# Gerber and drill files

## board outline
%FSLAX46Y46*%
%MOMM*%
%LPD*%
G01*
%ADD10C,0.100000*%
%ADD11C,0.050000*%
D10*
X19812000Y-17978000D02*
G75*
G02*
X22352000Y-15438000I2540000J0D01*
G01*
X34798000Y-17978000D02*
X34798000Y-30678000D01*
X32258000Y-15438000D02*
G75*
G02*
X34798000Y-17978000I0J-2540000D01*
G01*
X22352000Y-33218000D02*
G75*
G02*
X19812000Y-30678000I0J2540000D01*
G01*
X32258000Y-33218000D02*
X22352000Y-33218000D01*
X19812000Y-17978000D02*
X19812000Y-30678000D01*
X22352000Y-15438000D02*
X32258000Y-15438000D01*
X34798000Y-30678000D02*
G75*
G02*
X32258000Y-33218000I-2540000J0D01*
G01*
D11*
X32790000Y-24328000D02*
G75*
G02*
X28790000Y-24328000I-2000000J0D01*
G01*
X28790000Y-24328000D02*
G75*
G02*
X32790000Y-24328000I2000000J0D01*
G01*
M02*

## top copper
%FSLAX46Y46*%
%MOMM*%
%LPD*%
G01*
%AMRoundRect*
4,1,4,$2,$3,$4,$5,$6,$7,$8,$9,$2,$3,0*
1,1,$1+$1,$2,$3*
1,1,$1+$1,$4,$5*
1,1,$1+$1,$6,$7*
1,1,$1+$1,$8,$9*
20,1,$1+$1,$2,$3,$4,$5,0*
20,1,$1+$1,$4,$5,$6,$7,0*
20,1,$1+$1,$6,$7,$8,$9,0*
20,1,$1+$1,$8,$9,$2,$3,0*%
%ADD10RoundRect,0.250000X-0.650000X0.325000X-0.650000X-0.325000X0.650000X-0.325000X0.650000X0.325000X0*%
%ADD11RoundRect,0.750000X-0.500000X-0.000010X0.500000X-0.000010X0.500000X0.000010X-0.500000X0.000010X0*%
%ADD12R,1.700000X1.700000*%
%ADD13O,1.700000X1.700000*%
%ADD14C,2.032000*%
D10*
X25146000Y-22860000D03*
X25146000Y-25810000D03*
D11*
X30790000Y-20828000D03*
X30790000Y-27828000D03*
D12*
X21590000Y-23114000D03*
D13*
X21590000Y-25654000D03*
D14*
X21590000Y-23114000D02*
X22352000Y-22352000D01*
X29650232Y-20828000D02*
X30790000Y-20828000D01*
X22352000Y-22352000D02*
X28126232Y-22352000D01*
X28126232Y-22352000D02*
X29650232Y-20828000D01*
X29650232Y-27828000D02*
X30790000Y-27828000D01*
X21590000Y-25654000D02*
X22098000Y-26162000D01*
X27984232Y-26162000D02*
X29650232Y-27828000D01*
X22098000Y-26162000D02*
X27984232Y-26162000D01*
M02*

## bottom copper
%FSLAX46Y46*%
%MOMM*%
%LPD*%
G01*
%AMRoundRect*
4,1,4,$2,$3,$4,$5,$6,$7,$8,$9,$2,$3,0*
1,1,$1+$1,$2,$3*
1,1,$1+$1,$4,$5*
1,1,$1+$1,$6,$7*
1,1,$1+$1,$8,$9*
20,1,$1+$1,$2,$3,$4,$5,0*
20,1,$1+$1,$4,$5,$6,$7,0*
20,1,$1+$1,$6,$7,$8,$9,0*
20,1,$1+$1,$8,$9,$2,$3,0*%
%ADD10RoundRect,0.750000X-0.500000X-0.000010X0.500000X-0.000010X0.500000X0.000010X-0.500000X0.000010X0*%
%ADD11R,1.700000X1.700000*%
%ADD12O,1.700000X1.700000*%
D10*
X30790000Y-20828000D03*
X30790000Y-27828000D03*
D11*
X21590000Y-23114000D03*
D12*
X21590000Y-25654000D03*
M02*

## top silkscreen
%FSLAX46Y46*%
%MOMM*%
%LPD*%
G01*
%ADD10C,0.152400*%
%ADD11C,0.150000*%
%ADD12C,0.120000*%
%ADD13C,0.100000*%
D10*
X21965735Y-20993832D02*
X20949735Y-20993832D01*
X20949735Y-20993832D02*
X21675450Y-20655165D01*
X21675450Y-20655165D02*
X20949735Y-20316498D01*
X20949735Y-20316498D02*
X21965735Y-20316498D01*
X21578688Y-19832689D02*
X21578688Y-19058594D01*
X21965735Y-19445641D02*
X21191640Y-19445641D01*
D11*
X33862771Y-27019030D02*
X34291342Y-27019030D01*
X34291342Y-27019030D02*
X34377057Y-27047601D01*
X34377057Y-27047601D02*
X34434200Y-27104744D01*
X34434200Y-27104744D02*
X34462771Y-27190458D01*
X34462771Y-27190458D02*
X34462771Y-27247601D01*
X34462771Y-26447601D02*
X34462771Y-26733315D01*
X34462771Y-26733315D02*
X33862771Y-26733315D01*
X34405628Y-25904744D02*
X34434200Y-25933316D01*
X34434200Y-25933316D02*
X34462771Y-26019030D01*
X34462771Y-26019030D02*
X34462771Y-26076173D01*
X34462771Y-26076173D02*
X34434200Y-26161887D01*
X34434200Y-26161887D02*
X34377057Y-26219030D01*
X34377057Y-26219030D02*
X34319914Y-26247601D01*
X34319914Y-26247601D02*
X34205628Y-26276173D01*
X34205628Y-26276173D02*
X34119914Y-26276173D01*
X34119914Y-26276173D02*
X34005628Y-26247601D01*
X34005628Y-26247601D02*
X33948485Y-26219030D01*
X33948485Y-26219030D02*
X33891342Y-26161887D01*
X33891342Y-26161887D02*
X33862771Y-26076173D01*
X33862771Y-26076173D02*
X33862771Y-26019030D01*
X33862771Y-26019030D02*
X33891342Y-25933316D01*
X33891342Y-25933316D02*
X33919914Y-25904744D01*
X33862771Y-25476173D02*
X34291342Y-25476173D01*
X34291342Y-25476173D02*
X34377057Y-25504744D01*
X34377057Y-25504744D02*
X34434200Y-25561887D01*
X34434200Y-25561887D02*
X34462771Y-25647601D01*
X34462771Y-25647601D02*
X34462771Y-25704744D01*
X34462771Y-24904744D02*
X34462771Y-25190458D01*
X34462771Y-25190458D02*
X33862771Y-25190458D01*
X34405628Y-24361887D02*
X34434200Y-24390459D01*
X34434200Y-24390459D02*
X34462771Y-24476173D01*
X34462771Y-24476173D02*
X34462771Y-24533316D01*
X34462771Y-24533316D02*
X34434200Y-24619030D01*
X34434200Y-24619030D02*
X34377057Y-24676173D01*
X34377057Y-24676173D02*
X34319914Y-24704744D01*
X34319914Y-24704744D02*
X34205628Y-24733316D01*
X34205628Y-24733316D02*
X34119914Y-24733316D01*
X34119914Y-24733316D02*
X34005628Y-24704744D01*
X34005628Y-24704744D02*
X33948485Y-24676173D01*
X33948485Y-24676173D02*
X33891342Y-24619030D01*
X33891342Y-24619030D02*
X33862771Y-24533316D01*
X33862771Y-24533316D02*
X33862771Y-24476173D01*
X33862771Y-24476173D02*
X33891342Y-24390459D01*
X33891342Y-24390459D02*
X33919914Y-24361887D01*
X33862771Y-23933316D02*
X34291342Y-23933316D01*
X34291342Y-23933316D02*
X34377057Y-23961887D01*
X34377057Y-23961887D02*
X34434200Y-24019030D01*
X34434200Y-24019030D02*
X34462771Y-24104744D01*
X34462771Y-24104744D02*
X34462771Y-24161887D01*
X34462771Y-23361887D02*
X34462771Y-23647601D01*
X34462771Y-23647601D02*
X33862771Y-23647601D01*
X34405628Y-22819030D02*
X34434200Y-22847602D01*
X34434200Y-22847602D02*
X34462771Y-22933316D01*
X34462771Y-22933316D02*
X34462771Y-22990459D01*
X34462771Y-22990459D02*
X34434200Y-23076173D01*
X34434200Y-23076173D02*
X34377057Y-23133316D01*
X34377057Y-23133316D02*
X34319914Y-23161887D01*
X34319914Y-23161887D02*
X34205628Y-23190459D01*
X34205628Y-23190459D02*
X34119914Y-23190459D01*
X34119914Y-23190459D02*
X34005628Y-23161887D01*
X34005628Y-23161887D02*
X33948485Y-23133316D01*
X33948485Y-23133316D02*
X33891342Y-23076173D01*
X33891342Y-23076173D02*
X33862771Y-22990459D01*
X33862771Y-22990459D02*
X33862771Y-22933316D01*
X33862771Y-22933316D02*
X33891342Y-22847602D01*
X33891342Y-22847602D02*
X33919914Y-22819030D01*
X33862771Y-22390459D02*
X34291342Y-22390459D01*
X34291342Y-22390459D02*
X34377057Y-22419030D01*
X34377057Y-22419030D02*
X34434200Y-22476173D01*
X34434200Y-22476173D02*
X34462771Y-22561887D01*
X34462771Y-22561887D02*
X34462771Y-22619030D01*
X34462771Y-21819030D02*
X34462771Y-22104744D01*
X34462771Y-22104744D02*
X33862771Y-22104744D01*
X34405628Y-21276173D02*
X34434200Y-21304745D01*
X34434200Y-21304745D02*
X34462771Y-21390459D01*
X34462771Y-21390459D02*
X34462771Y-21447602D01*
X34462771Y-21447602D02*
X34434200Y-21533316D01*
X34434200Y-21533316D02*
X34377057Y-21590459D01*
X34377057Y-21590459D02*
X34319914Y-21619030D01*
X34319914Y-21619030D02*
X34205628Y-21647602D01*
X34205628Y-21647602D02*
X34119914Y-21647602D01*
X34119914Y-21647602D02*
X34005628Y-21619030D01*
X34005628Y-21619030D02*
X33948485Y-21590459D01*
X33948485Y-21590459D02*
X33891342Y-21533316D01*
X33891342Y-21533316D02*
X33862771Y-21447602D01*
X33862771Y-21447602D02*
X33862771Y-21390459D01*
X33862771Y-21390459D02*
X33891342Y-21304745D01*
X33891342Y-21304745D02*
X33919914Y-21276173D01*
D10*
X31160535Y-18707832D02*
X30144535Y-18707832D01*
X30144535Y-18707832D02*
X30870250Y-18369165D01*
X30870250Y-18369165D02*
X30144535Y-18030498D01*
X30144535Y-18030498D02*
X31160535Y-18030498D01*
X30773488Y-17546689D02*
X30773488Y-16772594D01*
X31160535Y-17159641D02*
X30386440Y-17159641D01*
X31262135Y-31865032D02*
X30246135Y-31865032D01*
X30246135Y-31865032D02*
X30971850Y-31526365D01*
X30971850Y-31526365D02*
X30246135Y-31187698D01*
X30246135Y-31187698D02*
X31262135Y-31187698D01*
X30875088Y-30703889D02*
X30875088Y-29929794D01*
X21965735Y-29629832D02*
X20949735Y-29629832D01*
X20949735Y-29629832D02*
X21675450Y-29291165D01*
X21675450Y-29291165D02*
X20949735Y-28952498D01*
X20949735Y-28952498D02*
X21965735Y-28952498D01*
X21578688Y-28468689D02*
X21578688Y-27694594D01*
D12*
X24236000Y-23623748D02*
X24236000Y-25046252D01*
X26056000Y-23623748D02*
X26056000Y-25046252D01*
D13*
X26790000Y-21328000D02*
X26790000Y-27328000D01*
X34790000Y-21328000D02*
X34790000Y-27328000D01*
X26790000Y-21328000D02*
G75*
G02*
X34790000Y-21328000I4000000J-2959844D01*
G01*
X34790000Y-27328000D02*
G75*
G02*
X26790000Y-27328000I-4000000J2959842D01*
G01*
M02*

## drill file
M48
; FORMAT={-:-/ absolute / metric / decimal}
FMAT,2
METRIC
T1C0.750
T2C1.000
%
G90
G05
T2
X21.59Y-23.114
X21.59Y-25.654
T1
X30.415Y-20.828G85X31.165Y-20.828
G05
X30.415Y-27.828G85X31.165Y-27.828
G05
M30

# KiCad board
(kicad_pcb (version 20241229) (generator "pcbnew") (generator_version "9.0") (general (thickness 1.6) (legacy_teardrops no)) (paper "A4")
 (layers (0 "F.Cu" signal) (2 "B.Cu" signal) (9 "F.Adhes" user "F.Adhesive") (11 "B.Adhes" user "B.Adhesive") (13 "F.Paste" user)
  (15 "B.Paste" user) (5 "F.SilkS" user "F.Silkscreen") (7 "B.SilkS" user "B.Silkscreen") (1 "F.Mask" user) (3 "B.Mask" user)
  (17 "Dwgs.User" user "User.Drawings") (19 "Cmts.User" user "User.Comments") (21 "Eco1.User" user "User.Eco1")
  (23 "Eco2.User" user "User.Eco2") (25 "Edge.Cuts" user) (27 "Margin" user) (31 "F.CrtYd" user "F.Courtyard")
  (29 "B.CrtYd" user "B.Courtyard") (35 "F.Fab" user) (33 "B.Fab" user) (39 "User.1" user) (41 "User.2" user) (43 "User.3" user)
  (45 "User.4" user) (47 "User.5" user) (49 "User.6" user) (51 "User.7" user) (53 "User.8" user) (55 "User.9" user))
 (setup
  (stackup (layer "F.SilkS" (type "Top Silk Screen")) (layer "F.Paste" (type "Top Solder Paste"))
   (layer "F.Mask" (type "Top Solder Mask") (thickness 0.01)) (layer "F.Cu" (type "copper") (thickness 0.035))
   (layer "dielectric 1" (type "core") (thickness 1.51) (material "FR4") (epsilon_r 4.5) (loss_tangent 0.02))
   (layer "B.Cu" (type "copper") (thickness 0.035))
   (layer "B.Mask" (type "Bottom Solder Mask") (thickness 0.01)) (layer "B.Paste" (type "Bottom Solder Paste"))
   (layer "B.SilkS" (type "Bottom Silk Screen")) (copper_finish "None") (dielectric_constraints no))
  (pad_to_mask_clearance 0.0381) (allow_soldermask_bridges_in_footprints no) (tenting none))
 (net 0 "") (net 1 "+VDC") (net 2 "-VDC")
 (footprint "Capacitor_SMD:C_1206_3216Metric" (layer "F.Cu") (at 25.146 24.335 -90)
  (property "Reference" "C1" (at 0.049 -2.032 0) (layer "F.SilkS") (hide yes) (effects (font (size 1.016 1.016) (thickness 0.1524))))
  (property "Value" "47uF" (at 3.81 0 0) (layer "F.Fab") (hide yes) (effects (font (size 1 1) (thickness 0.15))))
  (fp_line (start -0.711252 0.91) (end 0.711252 0.91) (stroke (width 0.12) (type solid)) (layer "F.SilkS"))
  (fp_line (start -0.711252 -0.91) (end 0.711252 -0.91) (stroke (width 0.12) (type solid)) (layer "F.SilkS"))
  (pad "1" smd roundrect (at -1.475 0 270) (size 1.15 1.8) (layers "F.Cu" "F.Mask" "F.Paste") (roundrect_rratio 0.2173913043) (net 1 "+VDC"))
  (pad "2" smd roundrect (at 1.475 0 270) (size 1.15 1.8) (layers "F.Cu" "F.Mask" "F.Paste") (roundrect_rratio 0.2173913043) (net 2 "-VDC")))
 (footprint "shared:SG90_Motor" (layer "F.Cu") (at 30.79 24.328)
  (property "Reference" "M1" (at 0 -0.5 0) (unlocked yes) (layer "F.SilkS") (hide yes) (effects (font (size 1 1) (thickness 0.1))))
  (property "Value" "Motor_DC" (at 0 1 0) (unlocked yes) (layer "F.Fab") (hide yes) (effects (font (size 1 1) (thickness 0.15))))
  (fp_line (start -4 -3) (end -4 3) (stroke (width 0.1) (type default)) (layer "F.SilkS"))
  (fp_line (start 4 -3) (end 4 3) (stroke (width 0.1) (type default)) (layer "F.SilkS"))
  (fp_arc (start -4 -3) (mid 0 -5.016166) (end 4 -3) (stroke (width 0.1) (type default)) (layer "F.SilkS"))
  (fp_arc (start 4 3) (mid 0 5.016167) (end -4 3) (stroke (width 0.1) (type default)) (layer "F.SilkS"))
  (fp_circle (center 0 0) (end 2 0) (stroke (width 0.05) (type default)) (fill no) (layer "Edge.Cuts"))
  (pad "1" thru_hole roundrect (at 0 -3.5) (size 2.5 1.5) (drill oval 1.5 0.75) (layers "*.Cu" "*.Mask") (remove_unused_layers no)
   (roundrect_rratio 0.5) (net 1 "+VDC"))
  (pad "2" thru_hole roundrect (at 0 3.5) (size 2.5 1.5) (drill oval 1.5 0.75) (layers "*.Cu" "*.Mask") (remove_unused_layers no)
   (roundrect_rratio 0.5) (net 2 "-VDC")))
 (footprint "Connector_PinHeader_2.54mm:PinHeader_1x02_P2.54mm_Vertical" (layer "B.Cu") (at 21.59 23.114 180)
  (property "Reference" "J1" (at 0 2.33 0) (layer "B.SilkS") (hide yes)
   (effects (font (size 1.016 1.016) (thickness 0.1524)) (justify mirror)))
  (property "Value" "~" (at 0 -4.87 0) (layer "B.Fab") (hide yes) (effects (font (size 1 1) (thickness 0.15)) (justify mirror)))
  (pad "1" thru_hole rect (at 0 0 180) (size 1.7 1.7) (drill 1) (layers "*.Cu" "*.Mask") (remove_unused_layers no) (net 1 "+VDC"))
  (pad "2" thru_hole oval (at 0 -2.54 180) (size 1.7 1.7) (drill 1) (layers "*.Cu" "*.Mask") (remove_unused_layers no) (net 2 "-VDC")))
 (gr_arc (start 19.812 17.978) (mid 20.555949 16.181949) (end 22.352 15.438) (stroke (width 0.1) (type default)) (layer "Edge.Cuts"))
 (gr_line (start 34.798 17.978) (end 34.798 30.678) (stroke (width 0.1) (type default)) (layer "Edge.Cuts"))
 (gr_arc (start 32.258 15.438) (mid 34.054051 16.181949) (end 34.798 17.978) (stroke (width 0.1) (type default)) (layer "Edge.Cuts"))
 (gr_arc (start 22.352 33.218) (mid 20.555949 32.474051) (end 19.812 30.678) (stroke (width 0.1) (type default)) (layer "Edge.Cuts"))
 (gr_line (start 32.258 33.218) (end 22.352 33.218) (stroke (width 0.1) (type default)) (layer "Edge.Cuts"))
 (gr_line (start 19.812 17.978) (end 19.812 30.678) (stroke (width 0.1) (type default)) (layer "Edge.Cuts"))
 (gr_line (start 22.352 15.438) (end 32.258 15.438) (stroke (width 0.1) (type default)) (layer "Edge.Cuts"))
 (gr_arc (start 34.798 30.678) (mid 34.054051 32.474051) (end 32.258 33.218) (stroke (width 0.1) (type default)) (layer "Edge.Cuts"))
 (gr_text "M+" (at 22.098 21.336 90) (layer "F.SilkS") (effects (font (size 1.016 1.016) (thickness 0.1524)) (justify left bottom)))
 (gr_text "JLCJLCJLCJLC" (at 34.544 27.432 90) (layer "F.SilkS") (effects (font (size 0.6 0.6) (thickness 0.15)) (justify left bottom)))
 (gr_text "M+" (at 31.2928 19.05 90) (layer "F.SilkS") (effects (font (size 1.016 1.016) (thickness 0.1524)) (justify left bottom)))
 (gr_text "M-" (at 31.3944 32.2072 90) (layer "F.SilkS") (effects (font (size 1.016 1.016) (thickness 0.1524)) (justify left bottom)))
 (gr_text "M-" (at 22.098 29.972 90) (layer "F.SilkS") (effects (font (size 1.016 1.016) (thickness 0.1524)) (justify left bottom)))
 (segment (start 21.59 23.114) (end 22.352 22.352) (width 2.032) (layer "F.Cu") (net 1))
 (segment (start 29.650232 20.828) (end 30.79 20.828) (width 2.032) (layer "F.Cu") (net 1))
 (segment (start 22.352 22.352) (end 28.126232 22.352) (width 2.032) (layer "F.Cu") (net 1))
 (segment (start 28.126232 22.352) (end 29.650232 20.828) (width 2.032) (layer "F.Cu") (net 1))
 (segment (start 29.650232 27.828) (end 30.79 27.828) (width 2.032) (layer "F.Cu") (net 2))
 (segment (start 21.59 25.654) (end 22.098 26.162) (width 2.032) (layer "F.Cu") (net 2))
 (segment (start 27.984232 26.162) (end 29.650232 27.828) (width 2.032) (layer "F.Cu") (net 2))
 (segment (start 22.098 26.162) (end 27.984232 26.162) (width 2.032) (layer "F.Cu") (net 2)))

